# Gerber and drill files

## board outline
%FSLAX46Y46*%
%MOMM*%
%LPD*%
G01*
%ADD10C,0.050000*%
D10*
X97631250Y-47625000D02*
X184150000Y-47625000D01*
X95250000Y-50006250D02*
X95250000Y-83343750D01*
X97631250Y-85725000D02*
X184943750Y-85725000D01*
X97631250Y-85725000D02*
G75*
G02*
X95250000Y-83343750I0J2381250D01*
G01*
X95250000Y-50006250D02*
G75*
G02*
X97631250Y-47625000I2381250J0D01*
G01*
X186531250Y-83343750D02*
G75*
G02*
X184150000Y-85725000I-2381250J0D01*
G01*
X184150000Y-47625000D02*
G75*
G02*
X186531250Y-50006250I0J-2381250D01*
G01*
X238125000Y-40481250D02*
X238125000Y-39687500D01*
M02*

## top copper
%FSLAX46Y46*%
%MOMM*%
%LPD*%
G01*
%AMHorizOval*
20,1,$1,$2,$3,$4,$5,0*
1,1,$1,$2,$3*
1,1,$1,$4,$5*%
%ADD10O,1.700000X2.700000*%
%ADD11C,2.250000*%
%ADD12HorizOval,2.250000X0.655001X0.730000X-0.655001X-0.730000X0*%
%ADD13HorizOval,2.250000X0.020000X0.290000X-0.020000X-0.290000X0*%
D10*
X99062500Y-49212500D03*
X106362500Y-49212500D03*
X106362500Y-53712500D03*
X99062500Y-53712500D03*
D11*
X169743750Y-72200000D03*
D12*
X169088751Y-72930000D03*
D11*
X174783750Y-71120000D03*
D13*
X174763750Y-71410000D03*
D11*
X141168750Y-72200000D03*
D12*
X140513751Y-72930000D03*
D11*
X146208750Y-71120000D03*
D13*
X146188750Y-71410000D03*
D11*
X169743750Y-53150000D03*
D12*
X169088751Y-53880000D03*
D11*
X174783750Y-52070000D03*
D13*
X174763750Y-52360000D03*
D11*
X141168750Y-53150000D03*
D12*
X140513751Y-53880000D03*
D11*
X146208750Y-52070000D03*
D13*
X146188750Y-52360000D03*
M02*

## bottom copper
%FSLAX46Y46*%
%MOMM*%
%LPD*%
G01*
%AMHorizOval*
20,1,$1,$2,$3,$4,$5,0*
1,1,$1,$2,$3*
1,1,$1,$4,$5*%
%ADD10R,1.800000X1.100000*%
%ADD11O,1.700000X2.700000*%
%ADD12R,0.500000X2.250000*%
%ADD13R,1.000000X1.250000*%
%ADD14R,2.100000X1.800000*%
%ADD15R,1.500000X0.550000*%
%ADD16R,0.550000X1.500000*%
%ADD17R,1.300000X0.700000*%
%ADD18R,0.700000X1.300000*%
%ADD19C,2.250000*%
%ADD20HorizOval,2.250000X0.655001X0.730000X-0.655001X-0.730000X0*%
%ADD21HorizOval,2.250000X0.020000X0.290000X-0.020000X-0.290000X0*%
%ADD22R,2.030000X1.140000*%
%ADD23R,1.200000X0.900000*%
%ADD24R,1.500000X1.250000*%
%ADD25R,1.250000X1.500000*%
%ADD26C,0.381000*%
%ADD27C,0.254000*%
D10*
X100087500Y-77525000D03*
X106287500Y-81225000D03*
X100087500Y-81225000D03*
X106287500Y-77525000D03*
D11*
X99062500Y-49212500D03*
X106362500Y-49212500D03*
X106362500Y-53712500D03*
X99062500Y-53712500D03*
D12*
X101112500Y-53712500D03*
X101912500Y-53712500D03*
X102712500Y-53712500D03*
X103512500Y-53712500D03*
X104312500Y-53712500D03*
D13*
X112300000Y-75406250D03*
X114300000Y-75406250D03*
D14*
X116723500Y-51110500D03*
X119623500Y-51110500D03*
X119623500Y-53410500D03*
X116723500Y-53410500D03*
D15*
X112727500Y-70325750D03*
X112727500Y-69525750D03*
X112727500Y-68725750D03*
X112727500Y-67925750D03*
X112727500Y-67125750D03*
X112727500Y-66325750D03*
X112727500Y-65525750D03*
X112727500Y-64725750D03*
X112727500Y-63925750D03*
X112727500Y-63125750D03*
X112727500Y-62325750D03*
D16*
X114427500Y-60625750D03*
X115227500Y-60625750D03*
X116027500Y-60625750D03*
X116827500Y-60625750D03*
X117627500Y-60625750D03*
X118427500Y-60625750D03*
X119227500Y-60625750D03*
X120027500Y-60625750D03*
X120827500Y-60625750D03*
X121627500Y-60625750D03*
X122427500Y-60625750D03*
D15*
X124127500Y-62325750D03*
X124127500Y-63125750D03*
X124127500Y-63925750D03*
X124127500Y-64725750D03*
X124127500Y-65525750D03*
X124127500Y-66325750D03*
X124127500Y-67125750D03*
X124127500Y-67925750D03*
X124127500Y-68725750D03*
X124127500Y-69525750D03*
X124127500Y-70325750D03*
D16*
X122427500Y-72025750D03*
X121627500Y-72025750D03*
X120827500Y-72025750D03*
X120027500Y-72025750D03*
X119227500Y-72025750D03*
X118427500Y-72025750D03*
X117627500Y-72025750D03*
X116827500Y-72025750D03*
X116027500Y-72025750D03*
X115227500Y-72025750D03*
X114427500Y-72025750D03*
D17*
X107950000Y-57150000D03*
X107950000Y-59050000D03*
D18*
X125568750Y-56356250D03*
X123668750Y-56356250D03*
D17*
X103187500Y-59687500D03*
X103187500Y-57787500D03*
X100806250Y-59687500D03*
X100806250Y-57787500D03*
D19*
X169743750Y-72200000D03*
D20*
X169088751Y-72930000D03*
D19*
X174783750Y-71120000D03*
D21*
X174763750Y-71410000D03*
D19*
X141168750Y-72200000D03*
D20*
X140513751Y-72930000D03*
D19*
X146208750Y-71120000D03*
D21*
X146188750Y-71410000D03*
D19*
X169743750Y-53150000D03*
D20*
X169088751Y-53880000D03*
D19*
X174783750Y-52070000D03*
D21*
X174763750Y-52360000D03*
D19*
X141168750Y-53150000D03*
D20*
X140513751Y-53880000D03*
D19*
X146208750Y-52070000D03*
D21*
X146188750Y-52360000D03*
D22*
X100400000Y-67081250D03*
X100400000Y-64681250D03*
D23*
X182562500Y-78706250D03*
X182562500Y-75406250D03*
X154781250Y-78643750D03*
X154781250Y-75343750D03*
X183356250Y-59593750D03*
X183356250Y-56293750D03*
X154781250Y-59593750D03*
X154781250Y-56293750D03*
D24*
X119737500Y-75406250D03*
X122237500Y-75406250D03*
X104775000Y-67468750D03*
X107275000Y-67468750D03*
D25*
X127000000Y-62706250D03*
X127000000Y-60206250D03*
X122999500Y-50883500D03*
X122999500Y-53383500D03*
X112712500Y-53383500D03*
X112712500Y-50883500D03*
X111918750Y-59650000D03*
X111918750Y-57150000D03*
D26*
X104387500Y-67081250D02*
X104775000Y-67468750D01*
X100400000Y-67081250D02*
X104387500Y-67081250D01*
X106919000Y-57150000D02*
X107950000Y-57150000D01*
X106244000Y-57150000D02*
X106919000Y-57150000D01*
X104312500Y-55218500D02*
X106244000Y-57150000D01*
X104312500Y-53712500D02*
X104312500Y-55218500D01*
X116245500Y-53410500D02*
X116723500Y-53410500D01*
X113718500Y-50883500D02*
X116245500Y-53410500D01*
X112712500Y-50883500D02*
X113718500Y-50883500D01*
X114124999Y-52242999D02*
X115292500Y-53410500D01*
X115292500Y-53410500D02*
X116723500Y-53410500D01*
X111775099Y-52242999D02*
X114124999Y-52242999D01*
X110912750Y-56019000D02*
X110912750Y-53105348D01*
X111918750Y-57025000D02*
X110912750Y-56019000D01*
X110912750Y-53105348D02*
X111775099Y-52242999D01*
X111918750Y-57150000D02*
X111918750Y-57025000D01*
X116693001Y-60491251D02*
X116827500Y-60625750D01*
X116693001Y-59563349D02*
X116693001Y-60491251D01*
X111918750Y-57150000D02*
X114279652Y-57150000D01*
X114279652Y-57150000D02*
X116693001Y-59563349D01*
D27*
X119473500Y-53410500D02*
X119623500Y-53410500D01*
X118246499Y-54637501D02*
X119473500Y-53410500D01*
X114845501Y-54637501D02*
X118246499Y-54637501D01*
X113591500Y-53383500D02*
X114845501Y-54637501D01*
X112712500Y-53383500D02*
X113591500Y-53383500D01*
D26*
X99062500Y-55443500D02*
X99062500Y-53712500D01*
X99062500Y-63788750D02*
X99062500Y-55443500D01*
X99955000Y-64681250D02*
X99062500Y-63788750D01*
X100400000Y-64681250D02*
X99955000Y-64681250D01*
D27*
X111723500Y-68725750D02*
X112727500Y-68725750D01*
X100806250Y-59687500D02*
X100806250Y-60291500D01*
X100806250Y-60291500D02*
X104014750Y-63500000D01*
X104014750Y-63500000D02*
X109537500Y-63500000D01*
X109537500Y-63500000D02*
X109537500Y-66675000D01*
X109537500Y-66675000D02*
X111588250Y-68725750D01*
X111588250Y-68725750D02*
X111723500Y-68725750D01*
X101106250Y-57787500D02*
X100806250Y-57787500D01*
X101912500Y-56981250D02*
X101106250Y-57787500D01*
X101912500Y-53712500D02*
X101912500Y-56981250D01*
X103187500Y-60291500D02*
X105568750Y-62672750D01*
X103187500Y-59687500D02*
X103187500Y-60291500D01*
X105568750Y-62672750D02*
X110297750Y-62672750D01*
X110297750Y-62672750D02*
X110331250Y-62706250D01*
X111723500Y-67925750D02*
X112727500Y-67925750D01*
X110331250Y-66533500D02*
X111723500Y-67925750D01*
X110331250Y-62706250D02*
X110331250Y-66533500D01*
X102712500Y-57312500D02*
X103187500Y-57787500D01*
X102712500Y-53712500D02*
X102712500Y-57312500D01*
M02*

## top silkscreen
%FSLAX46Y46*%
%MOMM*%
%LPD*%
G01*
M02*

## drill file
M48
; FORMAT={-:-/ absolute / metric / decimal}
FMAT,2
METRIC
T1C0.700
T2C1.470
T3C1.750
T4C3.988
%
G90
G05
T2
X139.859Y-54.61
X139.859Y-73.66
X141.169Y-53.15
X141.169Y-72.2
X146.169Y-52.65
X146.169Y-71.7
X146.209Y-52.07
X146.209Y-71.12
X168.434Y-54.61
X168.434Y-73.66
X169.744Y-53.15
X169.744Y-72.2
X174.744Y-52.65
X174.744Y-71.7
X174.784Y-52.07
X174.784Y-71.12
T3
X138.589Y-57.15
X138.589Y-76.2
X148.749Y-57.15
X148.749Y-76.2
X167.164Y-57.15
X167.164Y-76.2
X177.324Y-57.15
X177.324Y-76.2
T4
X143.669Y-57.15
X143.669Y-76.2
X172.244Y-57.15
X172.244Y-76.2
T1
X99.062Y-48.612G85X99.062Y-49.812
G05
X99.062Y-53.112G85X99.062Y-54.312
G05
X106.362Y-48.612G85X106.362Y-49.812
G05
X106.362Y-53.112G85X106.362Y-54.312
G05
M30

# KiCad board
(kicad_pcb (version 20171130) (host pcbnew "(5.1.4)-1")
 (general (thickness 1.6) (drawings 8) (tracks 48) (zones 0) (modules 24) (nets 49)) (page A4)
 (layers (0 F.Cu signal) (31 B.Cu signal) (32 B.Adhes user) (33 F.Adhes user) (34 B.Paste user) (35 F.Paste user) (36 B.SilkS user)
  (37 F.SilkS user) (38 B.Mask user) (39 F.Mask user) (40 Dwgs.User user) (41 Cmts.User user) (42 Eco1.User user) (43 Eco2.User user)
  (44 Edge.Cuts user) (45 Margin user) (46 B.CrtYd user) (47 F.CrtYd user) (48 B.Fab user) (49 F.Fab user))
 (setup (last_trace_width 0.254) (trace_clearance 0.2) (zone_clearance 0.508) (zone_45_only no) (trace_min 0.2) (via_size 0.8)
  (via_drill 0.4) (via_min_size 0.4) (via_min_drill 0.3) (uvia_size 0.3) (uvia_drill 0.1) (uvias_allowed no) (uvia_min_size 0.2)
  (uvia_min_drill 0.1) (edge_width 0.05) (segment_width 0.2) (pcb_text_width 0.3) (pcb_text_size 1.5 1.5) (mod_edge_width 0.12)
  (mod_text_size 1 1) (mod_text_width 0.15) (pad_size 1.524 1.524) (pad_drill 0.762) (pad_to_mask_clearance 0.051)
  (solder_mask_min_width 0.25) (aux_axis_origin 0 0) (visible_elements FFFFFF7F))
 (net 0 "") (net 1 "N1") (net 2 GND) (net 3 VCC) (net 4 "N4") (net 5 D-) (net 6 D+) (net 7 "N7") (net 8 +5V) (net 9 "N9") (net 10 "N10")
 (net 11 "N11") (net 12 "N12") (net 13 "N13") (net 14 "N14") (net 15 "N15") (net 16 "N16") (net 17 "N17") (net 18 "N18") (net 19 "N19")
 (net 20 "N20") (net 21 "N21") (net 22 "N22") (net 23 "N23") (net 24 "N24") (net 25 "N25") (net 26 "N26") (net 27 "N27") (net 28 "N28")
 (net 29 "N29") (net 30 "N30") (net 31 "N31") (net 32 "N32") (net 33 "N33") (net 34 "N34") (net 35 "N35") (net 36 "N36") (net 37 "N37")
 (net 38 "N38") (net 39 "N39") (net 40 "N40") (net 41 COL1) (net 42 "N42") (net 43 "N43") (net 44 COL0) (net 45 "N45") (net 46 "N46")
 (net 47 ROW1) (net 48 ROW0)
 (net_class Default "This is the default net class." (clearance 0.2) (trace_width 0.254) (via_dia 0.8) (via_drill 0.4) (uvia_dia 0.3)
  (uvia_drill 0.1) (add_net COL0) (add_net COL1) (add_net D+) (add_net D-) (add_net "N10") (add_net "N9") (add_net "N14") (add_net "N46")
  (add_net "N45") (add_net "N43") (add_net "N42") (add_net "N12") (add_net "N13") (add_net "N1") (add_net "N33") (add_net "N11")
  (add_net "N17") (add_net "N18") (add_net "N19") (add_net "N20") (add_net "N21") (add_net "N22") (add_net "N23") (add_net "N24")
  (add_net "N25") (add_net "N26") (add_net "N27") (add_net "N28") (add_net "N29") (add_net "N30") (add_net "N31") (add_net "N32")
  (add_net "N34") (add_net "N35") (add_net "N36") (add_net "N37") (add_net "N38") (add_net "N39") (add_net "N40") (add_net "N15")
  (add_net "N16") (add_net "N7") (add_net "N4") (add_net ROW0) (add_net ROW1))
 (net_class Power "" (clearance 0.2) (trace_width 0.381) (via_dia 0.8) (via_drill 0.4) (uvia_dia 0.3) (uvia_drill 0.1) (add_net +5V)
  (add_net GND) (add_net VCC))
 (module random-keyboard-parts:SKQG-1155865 (layer B.Cu) (at 103.1875 79.375)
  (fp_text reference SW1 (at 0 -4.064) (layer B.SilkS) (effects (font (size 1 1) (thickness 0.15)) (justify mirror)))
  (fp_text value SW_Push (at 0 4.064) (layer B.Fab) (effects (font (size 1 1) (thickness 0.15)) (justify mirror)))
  (pad 4 smd rect (at -3.1 -1.85) (size 1.8 1.1) (layers B.Cu B.Paste B.Mask))
  (pad 3 smd rect (at 3.1 1.85) (size 1.8 1.1) (layers B.Cu B.Paste B.Mask))
  (pad 2 smd rect (at -3.1 1.85) (size 1.8 1.1) (layers B.Cu B.Paste B.Mask) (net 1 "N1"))
  (pad 1 smd rect (at 3.1 -1.85) (size 1.8 1.1) (layers B.Cu B.Paste B.Mask) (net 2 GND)))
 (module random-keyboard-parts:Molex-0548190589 (layer B.Cu) (at 102.7125 49.2125 270)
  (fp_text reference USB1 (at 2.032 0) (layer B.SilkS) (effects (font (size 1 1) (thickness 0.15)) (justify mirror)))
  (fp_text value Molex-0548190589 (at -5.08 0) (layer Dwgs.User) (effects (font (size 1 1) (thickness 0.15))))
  (pad 6 thru_hole oval (at 0 3.65 270) (size 2.7 1.7) (drill oval 1.9 0.7) (layers *.Cu *.Mask) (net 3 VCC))
  (pad 6 thru_hole oval (at 0 -3.65 270) (size 2.7 1.7) (drill oval 1.9 0.7) (layers *.Cu *.Mask) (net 3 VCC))
  (pad 6 thru_hole oval (at 4.5 -3.65 270) (size 2.7 1.7) (drill oval 1.9 0.7) (layers *.Cu *.Mask) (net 3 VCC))
  (pad 6 thru_hole oval (at 4.5 3.65 270) (size 2.7 1.7) (drill oval 1.9 0.7) (layers *.Cu *.Mask) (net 3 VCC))
  (pad 5 smd rect (at 4.5 1.6 270) (size 2.25 0.5) (layers B.Cu B.Paste B.Mask) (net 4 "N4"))
  (pad 4 smd rect (at 4.5 0.8 270) (size 2.25 0.5) (layers B.Cu B.Paste B.Mask) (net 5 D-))
  (pad 3 smd rect (at 4.5 0 270) (size 2.25 0.5) (layers B.Cu B.Paste B.Mask) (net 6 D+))
  (pad 2 smd rect (at 4.5 -0.8 270) (size 2.25 0.5) (layers B.Cu B.Paste B.Mask) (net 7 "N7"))
  (pad 1 smd rect (at 4.5 -1.6 270) (size 2.25 0.5) (layers B.Cu B.Paste B.Mask) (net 2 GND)))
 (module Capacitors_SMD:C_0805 (layer B.Cu) (at 113.3 75.40625)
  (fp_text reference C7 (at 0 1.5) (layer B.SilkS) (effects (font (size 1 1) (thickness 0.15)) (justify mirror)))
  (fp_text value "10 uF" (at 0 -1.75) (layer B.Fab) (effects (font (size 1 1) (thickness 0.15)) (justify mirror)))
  (pad 1 smd rect (at -1 0) (size 1 1.25) (layers B.Cu B.Paste B.Mask) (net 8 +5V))
  (pad 2 smd rect (at 1 0) (size 1 1.25) (layers B.Cu B.Paste B.Mask) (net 2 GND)))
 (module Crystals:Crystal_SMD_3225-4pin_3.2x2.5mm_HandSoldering (layer B.Cu) (at 118.1735 52.2605)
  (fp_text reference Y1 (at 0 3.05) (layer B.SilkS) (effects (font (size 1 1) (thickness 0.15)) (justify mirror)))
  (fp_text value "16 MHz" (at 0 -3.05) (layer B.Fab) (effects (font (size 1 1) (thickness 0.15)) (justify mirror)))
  (pad 1 smd rect (at -1.45 -1.15) (size 2.1 1.8) (layers B.Cu B.Paste B.Mask) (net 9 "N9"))
  (pad 2 smd rect (at 1.45 -1.15) (size 2.1 1.8) (layers B.Cu B.Paste B.Mask) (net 2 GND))
  (pad 3 smd rect (at 1.45 1.15) (size 2.1 1.8) (layers B.Cu B.Paste B.Mask) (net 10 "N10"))
  (pad 4 smd rect (at -1.45 1.15) (size 2.1 1.8) (layers B.Cu B.Paste B.Mask) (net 2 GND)))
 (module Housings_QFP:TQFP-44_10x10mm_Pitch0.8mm (layer B.Cu) (at 118.4275 66.32575)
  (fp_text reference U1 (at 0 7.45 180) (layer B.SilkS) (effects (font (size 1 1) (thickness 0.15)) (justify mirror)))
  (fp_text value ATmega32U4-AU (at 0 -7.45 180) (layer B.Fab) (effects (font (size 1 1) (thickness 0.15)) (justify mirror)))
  (pad 1 smd rect (at -5.7 4) (size 1.5 0.55) (layers B.Cu B.Paste B.Mask) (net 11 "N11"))
  (pad 2 smd rect (at -5.7 3.2) (size 1.5 0.55) (layers B.Cu B.Paste B.Mask) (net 8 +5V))
  (pad 3 smd rect (at -5.7 2.4) (size 1.5 0.55) (layers B.Cu B.Paste B.Mask) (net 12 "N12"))
  (pad 4 smd rect (at -5.7 1.6) (size 1.5 0.55) (layers B.Cu B.Paste B.Mask) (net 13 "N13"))
  (pad 5 smd rect (at -5.7 0.8) (size 1.5 0.55) (layers B.Cu B.Paste B.Mask) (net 2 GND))
  (pad 6 smd rect (at -5.7 0) (size 1.5 0.55) (layers B.Cu B.Paste B.Mask) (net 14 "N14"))
  (pad 7 smd rect (at -5.7 -0.8) (size 1.5 0.55) (layers B.Cu B.Paste B.Mask) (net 8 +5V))
  (pad 8 smd rect (at -5.7 -1.6) (size 1.5 0.55) (layers B.Cu B.Paste B.Mask) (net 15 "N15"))
  (pad 9 smd rect (at -5.7 -2.4) (size 1.5 0.55) (layers B.Cu B.Paste B.Mask) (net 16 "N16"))
  (pad 10 smd rect (at -5.7 -3.2) (size 1.5 0.55) (layers B.Cu B.Paste B.Mask) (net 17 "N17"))
  (pad 11 smd rect (at -5.7 -4) (size 1.5 0.55) (layers B.Cu B.Paste B.Mask) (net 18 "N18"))
  (pad 12 smd rect (at -4 -5.7 270) (size 1.5 0.55) (layers B.Cu B.Paste B.Mask) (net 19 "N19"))
  (pad 13 smd rect (at -3.2 -5.7 270) (size 1.5 0.55) (layers B.Cu B.Paste B.Mask) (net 1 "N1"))
  (pad 14 smd rect (at -2.4 -5.7 270) (size 1.5 0.55) (layers B.Cu B.Paste B.Mask) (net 8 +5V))
  (pad 15 smd rect (at -1.6 -5.7 270) (size 1.5 0.55) (layers B.Cu B.Paste B.Mask) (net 2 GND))
  (pad 16 smd rect (at -0.8 -5.7 270) (size 1.5 0.55) (layers B.Cu B.Paste B.Mask) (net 10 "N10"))
  (pad 17 smd rect (at 0 -5.7 270) (size 1.5 0.55) (layers B.Cu B.Paste B.Mask) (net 9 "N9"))
  (pad 18 smd rect (at 0.8 -5.7 270) (size 1.5 0.55) (layers B.Cu B.Paste B.Mask) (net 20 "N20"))
  (pad 19 smd rect (at 1.6 -5.7 270) (size 1.5 0.55) (layers B.Cu B.Paste B.Mask) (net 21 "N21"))
  (pad 20 smd rect (at 2.4 -5.7 270) (size 1.5 0.55) (layers B.Cu B.Paste B.Mask) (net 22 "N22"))
  (pad 21 smd rect (at 3.2 -5.7 270) (size 1.5 0.55) (layers B.Cu B.Paste B.Mask) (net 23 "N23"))
  (pad 22 smd rect (at 4 -5.7 270) (size 1.5 0.55) (layers B.Cu B.Paste B.Mask) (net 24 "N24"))
  (pad 23 smd rect (at 5.7 -4) (size 1.5 0.55) (layers B.Cu B.Paste B.Mask) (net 2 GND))
  (pad 24 smd rect (at 5.7 -3.2) (size 1.5 0.55) (layers B.Cu B.Paste B.Mask) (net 8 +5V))
  (pad 25 smd rect (at 5.7 -2.4) (size 1.5 0.55) (layers B.Cu B.Paste B.Mask) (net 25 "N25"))
  (pad 26 smd rect (at 5.7 -1.6) (size 1.5 0.55) (layers B.Cu B.Paste B.Mask) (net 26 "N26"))
  (pad 27 smd rect (at 5.7 -0.8) (size 1.5 0.55) (layers B.Cu B.Paste B.Mask) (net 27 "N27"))
  (pad 28 smd rect (at 5.7 0) (size 1.5 0.55) (layers B.Cu B.Paste B.Mask) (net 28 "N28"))
  (pad 29 smd rect (at 5.7 0.8) (size 1.5 0.55) (layers B.Cu B.Paste B.Mask) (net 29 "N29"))
  (pad 30 smd rect (at 5.7 1.6) (size 1.5 0.55) (layers B.Cu B.Paste B.Mask) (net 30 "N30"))
  (pad 31 smd rect (at 5.7 2.4) (size 1.5 0.55) (layers B.Cu B.Paste B.Mask) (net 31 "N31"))
  (pad 32 smd rect (at 5.7 3.2) (size 1.5 0.55) (layers B.Cu B.Paste B.Mask) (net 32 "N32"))
  (pad 33 smd rect (at 5.7 4) (size 1.5 0.55) (layers B.Cu B.Paste B.Mask) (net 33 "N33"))
  (pad 34 smd rect (at 4 5.7 270) (size 1.5 0.55) (layers B.Cu B.Paste B.Mask) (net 8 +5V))
  (pad 35 smd rect (at 3.2 5.7 270) (size 1.5 0.55) (layers B.Cu B.Paste B.Mask) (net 2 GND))
  (pad 36 smd rect (at 2.4 5.7 270) (size 1.5 0.55) (layers B.Cu B.Paste B.Mask) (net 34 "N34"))
  (pad 37 smd rect (at 1.6 5.7 270) (size 1.5 0.55) (layers B.Cu B.Paste B.Mask) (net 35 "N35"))
  (pad 38 smd rect (at 0.8 5.7 270) (size 1.5 0.55) (layers B.Cu B.Paste B.Mask) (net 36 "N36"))
  (pad 39 smd rect (at 0 5.7 270) (size 1.5 0.55) (layers B.Cu B.Paste B.Mask) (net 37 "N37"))
  (pad 40 smd rect (at -0.8 5.7 270) (size 1.5 0.55) (layers B.Cu B.Paste B.Mask) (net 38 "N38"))
  (pad 41 smd rect (at -1.6 5.7 270) (size 1.5 0.55) (layers B.Cu B.Paste B.Mask) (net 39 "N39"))
  (pad 42 smd rect (at -2.4 5.7 270) (size 1.5 0.55) (layers B.Cu B.Paste B.Mask) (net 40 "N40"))
  (pad 43 smd rect (at -3.2 5.7 270) (size 1.5 0.55) (layers B.Cu B.Paste B.Mask) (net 2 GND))
  (pad 44 smd rect (at -4 5.7 270) (size 1.5 0.55) (layers B.Cu B.Paste B.Mask) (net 8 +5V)))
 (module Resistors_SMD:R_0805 (layer B.Cu) (at 107.95 58.1 270)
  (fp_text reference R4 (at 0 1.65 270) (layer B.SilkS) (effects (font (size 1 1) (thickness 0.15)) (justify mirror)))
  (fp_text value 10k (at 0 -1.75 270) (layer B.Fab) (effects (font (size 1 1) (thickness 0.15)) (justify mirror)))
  (pad 1 smd rect (at -0.95 0 270) (size 0.7 1.3) (layers B.Cu B.Paste B.Mask) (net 2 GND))
  (pad 2 smd rect (at 0.95 0 270) (size 0.7 1.3) (layers B.Cu B.Paste B.Mask) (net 33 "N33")))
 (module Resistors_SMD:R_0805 (layer B.Cu) (at 124.61875 56.35625 180)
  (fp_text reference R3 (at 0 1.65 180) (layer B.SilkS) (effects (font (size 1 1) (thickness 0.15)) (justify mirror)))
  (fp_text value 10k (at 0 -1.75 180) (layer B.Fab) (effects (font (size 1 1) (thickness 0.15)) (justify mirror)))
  (pad 1 smd rect (at -0.95 0 180) (size 0.7 1.3) (layers B.Cu B.Paste B.Mask) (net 8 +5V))
  (pad 2 smd rect (at 0.95 0 180) (size 0.7 1.3) (layers B.Cu B.Paste B.Mask) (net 1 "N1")))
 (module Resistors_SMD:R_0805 (layer B.Cu) (at 103.1875 58.7375 90)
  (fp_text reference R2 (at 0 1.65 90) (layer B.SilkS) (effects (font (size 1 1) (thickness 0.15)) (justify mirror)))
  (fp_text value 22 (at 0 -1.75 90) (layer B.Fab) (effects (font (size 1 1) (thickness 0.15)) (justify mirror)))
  (pad 1 smd rect (at -0.95 0 90) (size 0.7 1.3) (layers B.Cu B.Paste B.Mask) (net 13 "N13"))
  (pad 2 smd rect (at 0.95 0 90) (size 0.7 1.3) (layers B.Cu B.Paste B.Mask) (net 6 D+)))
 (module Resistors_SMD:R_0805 (layer B.Cu) (at 100.80625 58.7375 90)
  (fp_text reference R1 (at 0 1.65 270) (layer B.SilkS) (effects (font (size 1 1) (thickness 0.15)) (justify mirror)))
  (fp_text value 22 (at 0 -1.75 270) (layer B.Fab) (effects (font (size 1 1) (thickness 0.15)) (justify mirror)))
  (pad 1 smd rect (at -0.95 0 90) (size 0.7 1.3) (layers B.Cu B.Paste B.Mask) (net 12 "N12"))
  (pad 2 smd rect (at 0.95 0 90) (size 0.7 1.3) (layers B.Cu B.Paste B.Mask) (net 5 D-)))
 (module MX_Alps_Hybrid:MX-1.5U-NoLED (layer F.Cu) (at 172.24375 76.2)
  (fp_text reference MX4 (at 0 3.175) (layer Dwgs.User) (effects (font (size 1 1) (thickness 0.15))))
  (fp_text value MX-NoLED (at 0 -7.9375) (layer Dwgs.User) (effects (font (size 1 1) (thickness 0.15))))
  (pad "" np_thru_hole circle (at 5.08 0 48.0996) (size 1.75 1.75) (drill 1.75) (layers *.Cu *.Mask))
  (pad "" np_thru_hole circle (at -5.08 0 48.0996) (size 1.75 1.75) (drill 1.75) (layers *.Cu *.Mask))
  (pad 1 thru_hole circle (at -2.5 -4) (size 2.25 2.25) (drill 1.47) (layers *.Cu B.Mask) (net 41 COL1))
  (pad "" np_thru_hole circle (at 0 0) (size 3.9878 3.9878) (drill 3.9878) (layers *.Cu *.Mask))
  (pad 1 thru_hole oval (at -3.81 -2.54 48.0996) (size 4.211556 2.25) (drill 1.47 (offset 0.980778 0)) (layers *.Cu B.Mask) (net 41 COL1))
  (pad 2 thru_hole circle (at 2.54 -5.08) (size 2.25 2.25) (drill 1.47) (layers *.Cu B.Mask) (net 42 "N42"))
  (pad 2 thru_hole oval (at 2.5 -4.5 86.0548) (size 2.831378 2.25) (drill 1.47 (offset 0.290689 0)) (layers *.Cu B.Mask) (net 42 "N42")))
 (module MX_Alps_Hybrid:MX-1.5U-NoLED (layer F.Cu) (at 143.66875 76.2)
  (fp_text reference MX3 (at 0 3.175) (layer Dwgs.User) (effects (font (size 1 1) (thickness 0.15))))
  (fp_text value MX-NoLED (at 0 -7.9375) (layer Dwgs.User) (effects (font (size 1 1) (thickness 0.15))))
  (pad "" np_thru_hole circle (at 5.08 0 48.0996) (size 1.75 1.75) (drill 1.75) (layers *.Cu *.Mask))
  (pad "" np_thru_hole circle (at -5.08 0 48.0996) (size 1.75 1.75) (drill 1.75) (layers *.Cu *.Mask))
  (pad 1 thru_hole circle (at -2.5 -4) (size 2.25 2.25) (drill 1.47) (layers *.Cu B.Mask) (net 41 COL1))
  (pad "" np_thru_hole circle (at 0 0) (size 3.9878 3.9878) (drill 3.9878) (layers *.Cu *.Mask))
  (pad 1 thru_hole oval (at -3.81 -2.54 48.0996) (size 4.211556 2.25) (drill 1.47 (offset 0.980778 0)) (layers *.Cu B.Mask) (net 41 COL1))
  (pad 2 thru_hole circle (at 2.54 -5.08) (size 2.25 2.25) (drill 1.47) (layers *.Cu B.Mask) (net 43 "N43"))
  (pad 2 thru_hole oval (at 2.5 -4.5 86.0548) (size 2.831378 2.25) (drill 1.47 (offset 0.290689 0)) (layers *.Cu B.Mask) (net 43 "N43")))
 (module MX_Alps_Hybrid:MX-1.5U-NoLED (layer F.Cu) (at 172.24375 57.15)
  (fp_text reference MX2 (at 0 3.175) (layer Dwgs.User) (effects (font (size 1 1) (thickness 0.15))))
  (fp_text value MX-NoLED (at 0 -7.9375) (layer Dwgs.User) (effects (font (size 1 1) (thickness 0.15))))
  (pad "" np_thru_hole circle (at 5.08 0 48.0996) (size 1.75 1.75) (drill 1.75) (layers *.Cu *.Mask))
  (pad "" np_thru_hole circle (at -5.08 0 48.0996) (size 1.75 1.75) (drill 1.75) (layers *.Cu *.Mask))
  (pad 1 thru_hole circle (at -2.5 -4) (size 2.25 2.25) (drill 1.47) (layers *.Cu B.Mask) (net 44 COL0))
  (pad "" np_thru_hole circle (at 0 0) (size 3.9878 3.9878) (drill 3.9878) (layers *.Cu *.Mask))
  (pad 1 thru_hole oval (at -3.81 -2.54 48.0996) (size 4.211556 2.25) (drill 1.47 (offset 0.980778 0)) (layers *.Cu B.Mask) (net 44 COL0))
  (pad 2 thru_hole circle (at 2.54 -5.08) (size 2.25 2.25) (drill 1.47) (layers *.Cu B.Mask) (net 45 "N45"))
  (pad 2 thru_hole oval (at 2.5 -4.5 86.0548) (size 2.831378 2.25) (drill 1.47 (offset 0.290689 0)) (layers *.Cu B.Mask) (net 45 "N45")))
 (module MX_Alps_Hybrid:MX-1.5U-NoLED (layer F.Cu) (at 143.66875 57.15)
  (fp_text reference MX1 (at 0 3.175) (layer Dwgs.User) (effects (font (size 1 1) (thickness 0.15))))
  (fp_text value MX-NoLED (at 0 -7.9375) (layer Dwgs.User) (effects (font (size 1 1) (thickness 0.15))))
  (pad "" np_thru_hole circle (at 5.08 0 48.0996) (size 1.75 1.75) (drill 1.75) (layers *.Cu *.Mask))
  (pad "" np_thru_hole circle (at -5.08 0 48.0996) (size 1.75 1.75) (drill 1.75) (layers *.Cu *.Mask))
  (pad 1 thru_hole circle (at -2.5 -4) (size 2.25 2.25) (drill 1.47) (layers *.Cu B.Mask) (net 44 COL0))
  (pad "" np_thru_hole circle (at 0 0) (size 3.9878 3.9878) (drill 3.9878) (layers *.Cu *.Mask))
  (pad 1 thru_hole oval (at -3.81 -2.54 48.0996) (size 4.211556 2.25) (drill 1.47 (offset 0.980778 0)) (layers *.Cu B.Mask) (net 44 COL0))
  (pad 2 thru_hole circle (at 2.54 -5.08) (size 2.25 2.25) (drill 1.47) (layers *.Cu B.Mask) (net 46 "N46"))
  (pad 2 thru_hole oval (at 2.5 -4.5 86.0548) (size 2.831378 2.25) (drill 1.47 (offset 0.290689 0)) (layers *.Cu B.Mask) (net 46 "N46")))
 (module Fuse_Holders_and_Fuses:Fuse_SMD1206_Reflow (layer B.Cu) (at 100.4 65.88125 90)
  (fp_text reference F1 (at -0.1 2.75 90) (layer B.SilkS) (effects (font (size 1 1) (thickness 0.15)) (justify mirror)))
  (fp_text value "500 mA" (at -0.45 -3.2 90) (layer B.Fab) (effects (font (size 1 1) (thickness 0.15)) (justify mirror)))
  (pad 1 smd rect (at -1.2 0) (size 2.03 1.14) (layers B.Cu B.Paste B.Mask) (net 8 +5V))
  (pad 2 smd rect (at 1.2 0) (size 2.03 1.14) (layers B.Cu B.Paste B.Mask) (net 3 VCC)))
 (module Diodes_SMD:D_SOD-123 (layer B.Cu) (at 182.5625 77.05625 90)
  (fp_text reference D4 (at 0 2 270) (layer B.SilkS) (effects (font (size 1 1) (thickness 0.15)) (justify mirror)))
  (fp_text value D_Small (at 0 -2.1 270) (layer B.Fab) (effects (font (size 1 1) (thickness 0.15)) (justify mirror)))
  (pad 1 smd rect (at -1.65 0 90) (size 0.9 1.2) (layers B.Cu B.Paste B.Mask) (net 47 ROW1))
  (pad 2 smd rect (at 1.65 0 90) (size 0.9 1.2) (layers B.Cu B.Paste B.Mask) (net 42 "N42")))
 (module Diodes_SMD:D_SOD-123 (layer B.Cu) (at 154.78125 76.99375 90)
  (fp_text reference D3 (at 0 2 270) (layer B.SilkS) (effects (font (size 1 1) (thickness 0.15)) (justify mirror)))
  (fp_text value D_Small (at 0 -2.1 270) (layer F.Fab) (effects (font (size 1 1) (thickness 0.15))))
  (pad 1 smd rect (at -1.65 0 90) (size 0.9 1.2) (layers B.Cu B.Paste B.Mask) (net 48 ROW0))
  (pad 2 smd rect (at 1.65 0 90) (size 0.9 1.2) (layers B.Cu B.Paste B.Mask) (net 43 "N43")))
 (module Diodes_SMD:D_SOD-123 (layer B.Cu) (at 183.35625 57.94375 90)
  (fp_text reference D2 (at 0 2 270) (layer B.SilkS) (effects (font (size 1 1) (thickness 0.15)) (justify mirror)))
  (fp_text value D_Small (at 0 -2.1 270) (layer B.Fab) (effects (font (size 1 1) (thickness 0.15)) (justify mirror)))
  (pad 1 smd rect (at -1.65 0 90) (size 0.9 1.2) (layers B.Cu B.Paste B.Mask) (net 47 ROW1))
  (pad 2 smd rect (at 1.65 0 90) (size 0.9 1.2) (layers B.Cu B.Paste B.Mask) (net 45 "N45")))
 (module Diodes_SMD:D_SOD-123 (layer B.Cu) (at 154.78125 57.94375 90)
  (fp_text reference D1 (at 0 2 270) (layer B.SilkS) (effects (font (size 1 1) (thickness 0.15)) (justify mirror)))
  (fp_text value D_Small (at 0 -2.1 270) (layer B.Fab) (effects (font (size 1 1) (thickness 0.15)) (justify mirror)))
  (pad 1 smd rect (at -1.65 0 90) (size 0.9 1.2) (layers B.Cu B.Paste B.Mask) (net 48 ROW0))
  (pad 2 smd rect (at 1.65 0 90) (size 0.9 1.2) (layers B.Cu B.Paste B.Mask) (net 46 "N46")))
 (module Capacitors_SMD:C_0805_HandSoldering (layer B.Cu) (at 120.9875 75.40625)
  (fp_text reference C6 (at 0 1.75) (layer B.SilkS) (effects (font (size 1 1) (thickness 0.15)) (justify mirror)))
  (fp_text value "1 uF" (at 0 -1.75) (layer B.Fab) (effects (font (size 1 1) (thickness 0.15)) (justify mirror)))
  (pad 1 smd rect (at -1.25 0) (size 1.5 1.25) (layers B.Cu B.Paste B.Mask) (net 14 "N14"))
  (pad 2 smd rect (at 1.25 0) (size 1.5 1.25) (layers B.Cu B.Paste B.Mask) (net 2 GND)))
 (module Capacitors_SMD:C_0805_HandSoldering (layer B.Cu) (at 106.025 67.46875)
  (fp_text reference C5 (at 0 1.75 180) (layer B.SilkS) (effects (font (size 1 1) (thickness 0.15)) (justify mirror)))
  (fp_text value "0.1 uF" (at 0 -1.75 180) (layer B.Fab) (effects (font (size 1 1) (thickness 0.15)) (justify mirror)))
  (pad 1 smd rect (at -1.25 0) (size 1.5 1.25) (layers B.Cu B.Paste B.Mask) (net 8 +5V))
  (pad 2 smd rect (at 1.25 0) (size 1.5 1.25) (layers B.Cu B.Paste B.Mask) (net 2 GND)))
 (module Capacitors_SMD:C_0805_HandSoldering (layer B.Cu) (at 127 61.45625 90)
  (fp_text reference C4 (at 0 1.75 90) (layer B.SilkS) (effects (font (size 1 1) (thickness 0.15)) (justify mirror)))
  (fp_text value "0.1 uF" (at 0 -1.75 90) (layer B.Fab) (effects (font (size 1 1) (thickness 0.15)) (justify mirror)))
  (pad 1 smd rect (at -1.25 0 90) (size 1.5 1.25) (layers B.Cu B.Paste B.Mask) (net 8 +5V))
  (pad 2 smd rect (at 1.25 0 90) (size 1.5 1.25) (layers B.Cu B.Paste B.Mask) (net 2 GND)))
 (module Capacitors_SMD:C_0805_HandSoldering (layer B.Cu) (at 122.9995 52.1335 270)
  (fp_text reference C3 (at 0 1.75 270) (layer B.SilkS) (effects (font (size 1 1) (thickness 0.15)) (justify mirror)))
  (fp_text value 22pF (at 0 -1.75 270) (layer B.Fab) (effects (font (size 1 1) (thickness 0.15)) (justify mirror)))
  (pad 1 smd rect (at -1.25 0 270) (size 1.5 1.25) (layers B.Cu B.Paste B.Mask) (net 9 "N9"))
  (pad 2 smd rect (at 1.25 0 270) (size 1.5 1.25) (layers B.Cu B.Paste B.Mask) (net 2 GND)))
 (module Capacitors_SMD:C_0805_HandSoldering (layer B.Cu) (at 112.7125 52.1335 90)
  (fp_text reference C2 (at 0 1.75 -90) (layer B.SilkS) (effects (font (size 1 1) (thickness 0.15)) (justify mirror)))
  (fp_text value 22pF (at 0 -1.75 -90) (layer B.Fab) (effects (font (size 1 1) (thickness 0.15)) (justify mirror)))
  (pad 1 smd rect (at -1.25 0 90) (size 1.5 1.25) (layers B.Cu B.Paste B.Mask) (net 10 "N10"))
  (pad 2 smd rect (at 1.25 0 90) (size 1.5 1.25) (layers B.Cu B.Paste B.Mask) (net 2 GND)))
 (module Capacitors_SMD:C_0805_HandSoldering (layer B.Cu) (at 111.91875 58.4 90)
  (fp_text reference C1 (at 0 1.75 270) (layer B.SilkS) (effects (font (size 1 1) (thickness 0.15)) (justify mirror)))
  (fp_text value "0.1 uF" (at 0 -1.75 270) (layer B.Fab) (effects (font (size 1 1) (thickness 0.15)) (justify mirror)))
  (pad 1 smd rect (at -1.25 0 90) (size 1.5 1.25) (layers B.Cu B.Paste B.Mask) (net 8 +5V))
  (pad 2 smd rect (at 1.25 0 90) (size 1.5 1.25) (layers B.Cu B.Paste B.Mask) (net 2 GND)))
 (gr_line (start 97.63125 47.625) (end 184.15 47.625) (layer Edge.Cuts) (width 0.05))
 (gr_line (start 95.25 50.00625) (end 95.25 83.34375) (layer Edge.Cuts) (width 0.05))
 (gr_line (start 97.63125 85.725) (end 184.94375 85.725) (layer Edge.Cuts) (width 0.05))
 (gr_arc (start 97.63125 83.34375) (end 95.25 83.34375) (angle -90) (layer Edge.Cuts) (width 0.05))
 (gr_arc (start 97.63125 50.00625) (end 97.63125 47.625) (angle -90) (layer Edge.Cuts) (width 0.05))
 (gr_arc (start 184.15 83.34375) (end 184.15 85.725) (angle -90) (layer Edge.Cuts) (width 0.05))
 (gr_arc (start 184.15 50.00625) (end 186.53125 50.00625) (angle -90) (layer Edge.Cuts) (width 0.05))
 (gr_line (start 238.125 40.48125) (end 238.125 39.6875) (layer Edge.Cuts) (width 0.05))
 (segment (start 104.3875 67.08125) (end 104.775 67.46875) (width 0.381) (layer B.Cu) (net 8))
 (segment (start 100.4 67.08125) (end 104.3875 67.08125) (width 0.381) (layer B.Cu) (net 8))
 (segment (start 106.919 57.15) (end 107.95 57.15) (width 0.381) (layer B.Cu) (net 2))
 (segment (start 106.244 57.15) (end 106.919 57.15) (width 0.381) (layer B.Cu) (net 2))
 (segment (start 104.3125 55.2185) (end 106.244 57.15) (width 0.381) (layer B.Cu) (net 2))
 (segment (start 104.3125 53.7125) (end 104.3125 55.2185) (width 0.381) (layer B.Cu) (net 2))
 (segment (start 116.2455 53.4105) (end 116.7235 53.4105) (width 0.381) (layer B.Cu) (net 2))
 (segment (start 113.7185 50.8835) (end 116.2455 53.4105) (width 0.381) (layer B.Cu) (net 2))
 (segment (start 112.7125 50.8835) (end 113.7185 50.8835) (width 0.381) (layer B.Cu) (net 2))
 (segment (start 114.124999 52.242999) (end 115.2925 53.4105) (width 0.381) (layer B.Cu) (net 2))
 (segment (start 115.2925 53.4105) (end 116.7235 53.4105) (width 0.381) (layer B.Cu) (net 2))
 (segment (start 111.775099 52.242999) (end 114.124999 52.242999) (width 0.381) (layer B.Cu) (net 2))
 (segment (start 110.91275 56.019) (end 110.91275 53.105348) (width 0.381) (layer B.Cu) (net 2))
 (segment (start 111.91875 57.025) (end 110.91275 56.019) (width 0.381) (layer B.Cu) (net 2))
 (segment (start 110.91275 53.105348) (end 111.775099 52.242999) (width 0.381) (layer B.Cu) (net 2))
 (segment (start 111.91875 57.15) (end 111.91875 57.025) (width 0.381) (layer B.Cu) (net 2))
 (segment (start 116.693001 60.491251) (end 116.8275 60.62575) (width 0.381) (layer B.Cu) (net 2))
 (segment (start 116.693001 59.563349) (end 116.693001 60.491251) (width 0.381) (layer B.Cu) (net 2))
 (segment (start 111.91875 57.15) (end 114.279652 57.15) (width 0.381) (layer B.Cu) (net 2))
 (segment (start 114.279652 57.15) (end 116.693001 59.563349) (width 0.381) (layer B.Cu) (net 2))
 (segment (start 119.4735 53.4105) (end 119.6235 53.4105) (width 0.254) (layer B.Cu) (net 10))
 (segment (start 118.246499 54.637501) (end 119.4735 53.4105) (width 0.254) (layer B.Cu) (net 10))
 (segment (start 114.845501 54.637501) (end 118.246499 54.637501) (width 0.254) (layer B.Cu) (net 10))
 (segment (start 113.5915 53.3835) (end 114.845501 54.637501) (width 0.254) (layer B.Cu) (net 10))
 (segment (start 112.7125 53.3835) (end 113.5915 53.3835) (width 0.254) (layer B.Cu) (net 10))
 (segment (start 99.0625 55.4435) (end 99.0625 53.7125) (width 0.381) (layer B.Cu) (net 3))
 (segment (start 99.0625 63.78875) (end 99.0625 55.4435) (width 0.381) (layer B.Cu) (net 3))
 (segment (start 99.955 64.68125) (end 99.0625 63.78875) (width 0.381) (layer B.Cu) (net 3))
 (segment (start 100.4 64.68125) (end 99.955 64.68125) (width 0.381) (layer B.Cu) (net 3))
 (segment (start 111.7235 68.72575) (end 112.7275 68.72575) (width 0.254) (layer B.Cu) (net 12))
 (segment (start 100.80625 59.6875) (end 100.80625 60.2915) (width 0.254) (layer B.Cu) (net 12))
 (segment (start 100.80625 60.2915) (end 104.01475 63.5) (width 0.254) (layer B.Cu) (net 12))
 (segment (start 104.01475 63.5) (end 109.5375 63.5) (width 0.254) (layer B.Cu) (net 12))
 (segment (start 109.5375 63.5) (end 109.5375 66.675) (width 0.254) (layer B.Cu) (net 12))
 (segment (start 109.5375 66.675) (end 111.58825 68.72575) (width 0.254) (layer B.Cu) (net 12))
 (segment (start 111.58825 68.72575) (end 111.7235 68.72575) (width 0.254) (layer B.Cu) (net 12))
 (segment (start 101.10625 57.7875) (end 100.80625 57.7875) (width 0.254) (layer B.Cu) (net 5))
 (segment (start 101.9125 56.98125) (end 101.10625 57.7875) (width 0.254) (layer B.Cu) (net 5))
 (segment (start 101.9125 53.7125) (end 101.9125 56.98125) (width 0.254) (layer B.Cu) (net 5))
 (segment (start 103.1875 60.2915) (end 105.56875 62.67275) (width 0.254) (layer B.Cu) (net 13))
 (segment (start 103.1875 59.6875) (end 103.1875 60.2915) (width 0.254) (layer B.Cu) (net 13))
 (segment (start 105.56875 62.67275) (end 110.29775 62.67275) (width 0.254) (layer B.Cu) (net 13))
 (segment (start 110.29775 62.67275) (end 110.33125 62.70625) (width 0.254) (layer B.Cu) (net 13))
 (segment (start 111.7235 67.92575) (end 112.7275 67.92575) (width 0.254) (layer B.Cu) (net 13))
 (segment (start 110.33125 66.5335) (end 111.7235 67.92575) (width 0.254) (layer B.Cu) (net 13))
 (segment (start 110.33125 62.70625) (end 110.33125 66.5335) (width 0.254) (layer B.Cu) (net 13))
 (segment (start 102.7125 57.3125) (end 103.1875 57.7875) (width 0.254) (layer B.Cu) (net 6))
 (segment (start 102.7125 53.7125) (end 102.7125 57.3125) (width 0.254) (layer B.Cu) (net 6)))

